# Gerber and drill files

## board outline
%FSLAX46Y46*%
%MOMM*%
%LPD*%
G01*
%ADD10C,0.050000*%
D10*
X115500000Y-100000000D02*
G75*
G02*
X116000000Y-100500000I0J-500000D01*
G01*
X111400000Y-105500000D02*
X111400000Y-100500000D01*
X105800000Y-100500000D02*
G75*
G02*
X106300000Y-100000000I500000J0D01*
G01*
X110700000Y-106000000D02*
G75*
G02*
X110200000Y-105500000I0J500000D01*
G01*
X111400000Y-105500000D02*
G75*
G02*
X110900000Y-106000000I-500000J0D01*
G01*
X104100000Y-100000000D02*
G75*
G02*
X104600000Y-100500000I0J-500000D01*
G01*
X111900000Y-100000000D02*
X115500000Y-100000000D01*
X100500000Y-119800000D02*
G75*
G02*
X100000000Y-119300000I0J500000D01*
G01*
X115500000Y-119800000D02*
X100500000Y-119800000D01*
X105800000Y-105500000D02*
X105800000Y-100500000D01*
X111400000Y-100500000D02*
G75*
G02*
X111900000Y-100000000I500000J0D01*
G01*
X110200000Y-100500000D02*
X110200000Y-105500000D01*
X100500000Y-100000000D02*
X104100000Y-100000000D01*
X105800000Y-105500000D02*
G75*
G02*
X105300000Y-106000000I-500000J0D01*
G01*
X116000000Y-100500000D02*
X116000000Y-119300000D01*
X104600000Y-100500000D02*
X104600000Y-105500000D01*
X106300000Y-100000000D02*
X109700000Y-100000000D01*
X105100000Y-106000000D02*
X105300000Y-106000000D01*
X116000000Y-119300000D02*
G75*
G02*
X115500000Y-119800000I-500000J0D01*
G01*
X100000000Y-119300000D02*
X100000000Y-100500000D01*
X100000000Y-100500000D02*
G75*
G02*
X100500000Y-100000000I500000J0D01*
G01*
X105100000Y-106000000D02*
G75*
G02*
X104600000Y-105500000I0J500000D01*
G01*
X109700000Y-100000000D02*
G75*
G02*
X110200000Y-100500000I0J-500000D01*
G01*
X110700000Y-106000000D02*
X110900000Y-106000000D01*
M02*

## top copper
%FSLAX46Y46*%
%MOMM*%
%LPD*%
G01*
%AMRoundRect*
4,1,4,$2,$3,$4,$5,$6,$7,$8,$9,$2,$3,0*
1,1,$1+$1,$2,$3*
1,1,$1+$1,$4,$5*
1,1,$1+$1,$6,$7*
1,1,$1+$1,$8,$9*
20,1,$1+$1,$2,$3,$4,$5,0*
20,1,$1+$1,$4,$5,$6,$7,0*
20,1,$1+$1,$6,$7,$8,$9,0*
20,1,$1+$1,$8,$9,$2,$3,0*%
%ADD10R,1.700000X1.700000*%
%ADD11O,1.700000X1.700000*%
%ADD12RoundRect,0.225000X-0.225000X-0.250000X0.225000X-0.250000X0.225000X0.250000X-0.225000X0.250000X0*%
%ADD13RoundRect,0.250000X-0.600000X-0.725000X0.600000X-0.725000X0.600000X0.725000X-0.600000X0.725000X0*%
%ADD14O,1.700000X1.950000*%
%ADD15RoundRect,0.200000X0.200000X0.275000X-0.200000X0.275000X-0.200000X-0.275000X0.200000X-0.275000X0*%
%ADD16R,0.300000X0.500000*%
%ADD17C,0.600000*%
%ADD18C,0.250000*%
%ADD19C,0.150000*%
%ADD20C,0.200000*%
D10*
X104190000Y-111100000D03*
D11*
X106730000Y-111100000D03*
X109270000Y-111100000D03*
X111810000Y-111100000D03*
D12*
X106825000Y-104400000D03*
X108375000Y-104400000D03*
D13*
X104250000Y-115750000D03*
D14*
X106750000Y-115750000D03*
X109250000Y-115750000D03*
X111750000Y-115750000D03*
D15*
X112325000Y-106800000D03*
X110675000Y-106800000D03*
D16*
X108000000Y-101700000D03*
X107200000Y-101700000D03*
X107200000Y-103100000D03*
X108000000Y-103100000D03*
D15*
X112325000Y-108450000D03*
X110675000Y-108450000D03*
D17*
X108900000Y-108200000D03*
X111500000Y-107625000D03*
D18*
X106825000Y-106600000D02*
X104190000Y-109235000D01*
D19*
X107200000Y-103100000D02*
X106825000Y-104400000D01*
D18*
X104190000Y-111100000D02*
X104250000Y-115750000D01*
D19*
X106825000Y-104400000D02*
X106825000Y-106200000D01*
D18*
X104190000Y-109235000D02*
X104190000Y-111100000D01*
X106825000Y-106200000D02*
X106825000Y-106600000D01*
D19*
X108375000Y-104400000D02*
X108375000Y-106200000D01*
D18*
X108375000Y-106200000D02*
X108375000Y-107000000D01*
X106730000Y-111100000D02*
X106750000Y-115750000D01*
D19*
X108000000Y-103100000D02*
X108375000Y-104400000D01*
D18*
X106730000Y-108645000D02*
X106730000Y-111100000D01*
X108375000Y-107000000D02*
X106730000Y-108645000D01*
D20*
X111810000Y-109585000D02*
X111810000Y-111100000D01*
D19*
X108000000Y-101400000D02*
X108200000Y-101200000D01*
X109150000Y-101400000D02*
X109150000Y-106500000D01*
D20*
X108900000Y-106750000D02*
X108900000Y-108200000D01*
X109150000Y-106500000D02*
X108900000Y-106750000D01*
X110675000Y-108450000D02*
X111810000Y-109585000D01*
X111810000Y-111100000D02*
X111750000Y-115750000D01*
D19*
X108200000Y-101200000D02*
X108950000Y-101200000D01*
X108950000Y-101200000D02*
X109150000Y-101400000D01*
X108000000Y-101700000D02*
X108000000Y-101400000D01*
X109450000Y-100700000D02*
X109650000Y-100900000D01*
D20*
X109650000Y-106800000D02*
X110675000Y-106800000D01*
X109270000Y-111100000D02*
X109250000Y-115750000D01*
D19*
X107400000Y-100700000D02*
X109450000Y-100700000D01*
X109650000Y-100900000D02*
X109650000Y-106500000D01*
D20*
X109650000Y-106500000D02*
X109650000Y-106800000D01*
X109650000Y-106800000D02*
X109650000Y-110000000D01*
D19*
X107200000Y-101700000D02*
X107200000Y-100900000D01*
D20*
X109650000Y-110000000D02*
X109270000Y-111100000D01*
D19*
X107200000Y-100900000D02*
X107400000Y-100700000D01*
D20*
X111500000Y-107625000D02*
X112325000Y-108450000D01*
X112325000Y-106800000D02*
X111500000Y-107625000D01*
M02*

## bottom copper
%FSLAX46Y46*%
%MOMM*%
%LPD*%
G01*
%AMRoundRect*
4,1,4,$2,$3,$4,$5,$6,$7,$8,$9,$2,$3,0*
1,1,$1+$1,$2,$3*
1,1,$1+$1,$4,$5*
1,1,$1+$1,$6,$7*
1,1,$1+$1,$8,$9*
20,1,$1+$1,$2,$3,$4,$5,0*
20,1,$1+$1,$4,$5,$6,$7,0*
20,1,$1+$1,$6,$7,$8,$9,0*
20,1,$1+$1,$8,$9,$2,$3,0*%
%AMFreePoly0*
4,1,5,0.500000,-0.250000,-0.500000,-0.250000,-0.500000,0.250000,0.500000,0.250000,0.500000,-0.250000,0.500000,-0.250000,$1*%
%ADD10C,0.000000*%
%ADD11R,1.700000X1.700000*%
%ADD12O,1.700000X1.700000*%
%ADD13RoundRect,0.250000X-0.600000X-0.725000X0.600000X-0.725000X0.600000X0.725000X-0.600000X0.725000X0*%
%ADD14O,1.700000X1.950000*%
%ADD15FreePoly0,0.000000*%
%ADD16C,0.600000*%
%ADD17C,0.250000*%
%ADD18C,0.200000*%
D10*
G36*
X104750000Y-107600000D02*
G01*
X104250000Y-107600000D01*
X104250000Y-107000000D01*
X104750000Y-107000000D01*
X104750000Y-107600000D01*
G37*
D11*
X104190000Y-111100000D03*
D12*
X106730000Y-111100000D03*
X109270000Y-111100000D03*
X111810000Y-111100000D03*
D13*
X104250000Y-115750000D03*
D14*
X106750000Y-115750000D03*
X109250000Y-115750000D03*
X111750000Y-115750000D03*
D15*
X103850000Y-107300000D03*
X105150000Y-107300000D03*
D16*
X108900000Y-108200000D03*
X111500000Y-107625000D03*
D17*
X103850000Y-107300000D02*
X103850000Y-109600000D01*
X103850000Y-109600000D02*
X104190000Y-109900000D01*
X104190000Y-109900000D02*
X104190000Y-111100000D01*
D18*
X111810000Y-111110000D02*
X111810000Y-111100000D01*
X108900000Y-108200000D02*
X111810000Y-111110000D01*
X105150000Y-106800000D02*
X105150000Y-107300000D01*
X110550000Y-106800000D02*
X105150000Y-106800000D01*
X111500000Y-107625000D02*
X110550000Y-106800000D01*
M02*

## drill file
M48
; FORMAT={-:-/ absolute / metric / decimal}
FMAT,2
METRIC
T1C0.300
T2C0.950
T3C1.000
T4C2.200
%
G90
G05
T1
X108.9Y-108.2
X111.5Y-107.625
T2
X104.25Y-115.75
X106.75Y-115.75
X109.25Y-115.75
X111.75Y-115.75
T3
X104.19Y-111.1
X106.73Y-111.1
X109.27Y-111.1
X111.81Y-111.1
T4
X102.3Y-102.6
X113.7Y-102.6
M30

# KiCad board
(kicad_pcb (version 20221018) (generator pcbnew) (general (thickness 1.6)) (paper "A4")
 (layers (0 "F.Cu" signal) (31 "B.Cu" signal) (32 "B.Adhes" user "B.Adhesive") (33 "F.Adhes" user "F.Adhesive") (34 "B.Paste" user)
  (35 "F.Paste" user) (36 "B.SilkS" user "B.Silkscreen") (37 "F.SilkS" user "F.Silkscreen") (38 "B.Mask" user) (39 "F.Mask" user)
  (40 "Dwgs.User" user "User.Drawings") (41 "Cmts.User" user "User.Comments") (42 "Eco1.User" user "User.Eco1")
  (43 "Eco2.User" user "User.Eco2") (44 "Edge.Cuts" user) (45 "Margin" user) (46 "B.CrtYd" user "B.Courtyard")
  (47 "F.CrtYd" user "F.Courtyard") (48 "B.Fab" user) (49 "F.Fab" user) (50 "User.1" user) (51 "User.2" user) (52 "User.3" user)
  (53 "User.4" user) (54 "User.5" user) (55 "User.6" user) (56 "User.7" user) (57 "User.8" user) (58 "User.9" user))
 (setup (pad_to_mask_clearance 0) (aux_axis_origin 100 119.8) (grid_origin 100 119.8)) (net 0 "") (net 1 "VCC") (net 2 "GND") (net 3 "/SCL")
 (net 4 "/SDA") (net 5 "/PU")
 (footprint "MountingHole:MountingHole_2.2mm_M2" (layer "F.Cu") (at 113.7 102.6)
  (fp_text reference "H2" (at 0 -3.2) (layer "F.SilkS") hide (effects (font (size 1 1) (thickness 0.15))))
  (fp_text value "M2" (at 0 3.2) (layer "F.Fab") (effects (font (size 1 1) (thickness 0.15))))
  (pad "" np_thru_hole circle (at 0 0) (size 2.2 2.2) (drill 2.2) (layers "*.Cu" "*.Mask")))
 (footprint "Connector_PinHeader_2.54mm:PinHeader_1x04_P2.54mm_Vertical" (layer "F.Cu") (at 104.19 111.1 90)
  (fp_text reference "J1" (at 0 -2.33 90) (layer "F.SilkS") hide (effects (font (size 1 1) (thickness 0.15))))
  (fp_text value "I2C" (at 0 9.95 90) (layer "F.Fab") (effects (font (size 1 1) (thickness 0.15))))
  (pad "1" thru_hole rect (at 0 0 90) (size 1.7 1.7) (drill 1) (layers "*.Cu" "*.Mask") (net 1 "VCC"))
  (pad "2" thru_hole oval (at 0 2.54 90) (size 1.7 1.7) (drill 1) (layers "*.Cu" "*.Mask") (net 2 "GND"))
  (pad "3" thru_hole oval (at 0 5.08 90) (size 1.7 1.7) (drill 1) (layers "*.Cu" "*.Mask") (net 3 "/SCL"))
  (pad "4" thru_hole oval (at 0 7.62 90) (size 1.7 1.7) (drill 1) (layers "*.Cu" "*.Mask") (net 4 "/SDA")))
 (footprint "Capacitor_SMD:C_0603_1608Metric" (layer "F.Cu") (at 107.6 104.4)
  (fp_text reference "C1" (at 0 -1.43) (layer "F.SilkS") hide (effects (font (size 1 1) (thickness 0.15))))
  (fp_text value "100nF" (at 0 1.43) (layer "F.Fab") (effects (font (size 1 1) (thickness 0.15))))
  (pad "1" smd roundrect (at -0.775 0) (size 0.9 0.95) (layers "F.Cu" "F.Paste" "F.Mask") (roundrect_rratio 0.25) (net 1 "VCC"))
  (pad "2" smd roundrect (at 0.775 0) (size 0.9 0.95) (layers "F.Cu" "F.Paste" "F.Mask") (roundrect_rratio 0.25) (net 2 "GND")))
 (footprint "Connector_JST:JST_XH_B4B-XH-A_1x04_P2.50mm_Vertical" (layer "F.Cu") (at 104.25 115.75)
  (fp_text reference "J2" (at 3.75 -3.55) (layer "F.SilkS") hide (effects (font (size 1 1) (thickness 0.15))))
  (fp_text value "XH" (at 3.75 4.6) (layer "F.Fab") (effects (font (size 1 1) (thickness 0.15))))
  (pad "1" thru_hole roundrect (at 0 0) (size 1.7 1.95) (drill 0.95) (layers "*.Cu" "*.Mask") (roundrect_rratio 0.147059) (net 1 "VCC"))
  (pad "2" thru_hole oval (at 2.5 0) (size 1.7 1.95) (drill 0.95) (layers "*.Cu" "*.Mask") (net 2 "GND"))
  (pad "3" thru_hole oval (at 5 0) (size 1.7 1.95) (drill 0.95) (layers "*.Cu" "*.Mask") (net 3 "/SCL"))
  (pad "4" thru_hole oval (at 7.5 0) (size 1.7 1.95) (drill 0.95) (layers "*.Cu" "*.Mask") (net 4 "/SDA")))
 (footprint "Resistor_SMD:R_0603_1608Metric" (layer "F.Cu") (at 111.5 106.8 180)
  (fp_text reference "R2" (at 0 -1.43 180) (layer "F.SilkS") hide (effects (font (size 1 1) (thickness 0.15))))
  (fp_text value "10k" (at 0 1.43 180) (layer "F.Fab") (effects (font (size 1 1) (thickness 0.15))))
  (pad "1" smd roundrect (at -0.825 0 180) (size 0.8 0.95) (layers "F.Cu" "F.Paste" "F.Mask") (roundrect_rratio 0.25) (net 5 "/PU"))
  (pad "2" smd roundrect (at 0.825 0 180) (size 0.8 0.95) (layers "F.Cu" "F.Paste" "F.Mask") (roundrect_rratio 0.25) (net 3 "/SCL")))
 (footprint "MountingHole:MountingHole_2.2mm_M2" (layer "F.Cu") (at 102.3 102.6)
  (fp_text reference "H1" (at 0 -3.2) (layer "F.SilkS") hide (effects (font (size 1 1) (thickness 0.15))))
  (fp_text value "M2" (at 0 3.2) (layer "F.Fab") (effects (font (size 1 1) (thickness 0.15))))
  (pad "" np_thru_hole circle (at 0 0) (size 2.2 2.2) (drill 2.2) (layers "*.Cu" "*.Mask")))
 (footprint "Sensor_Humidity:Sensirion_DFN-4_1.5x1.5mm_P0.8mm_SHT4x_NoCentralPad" (layer "F.Cu") (at 107.6 102.4 -90)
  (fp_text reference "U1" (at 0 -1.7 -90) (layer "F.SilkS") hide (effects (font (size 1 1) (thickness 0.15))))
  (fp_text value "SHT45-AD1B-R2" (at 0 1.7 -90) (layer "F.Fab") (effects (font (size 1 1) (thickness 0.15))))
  (pad "1" smd rect (at -0.7 -0.4 270) (size 0.5 0.3) (layers "F.Cu" "F.Paste" "F.Mask") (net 4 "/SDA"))
  (pad "2" smd rect (at -0.7 0.4 270) (size 0.5 0.3) (layers "F.Cu" "F.Paste" "F.Mask") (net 3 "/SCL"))
  (pad "3" smd rect (at 0.7 0.4 270) (size 0.5 0.3) (layers "F.Cu" "F.Paste" "F.Mask") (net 1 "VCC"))
  (pad "4" smd rect (at 0.7 -0.4 270) (size 0.5 0.3) (layers "F.Cu" "F.Paste" "F.Mask") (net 2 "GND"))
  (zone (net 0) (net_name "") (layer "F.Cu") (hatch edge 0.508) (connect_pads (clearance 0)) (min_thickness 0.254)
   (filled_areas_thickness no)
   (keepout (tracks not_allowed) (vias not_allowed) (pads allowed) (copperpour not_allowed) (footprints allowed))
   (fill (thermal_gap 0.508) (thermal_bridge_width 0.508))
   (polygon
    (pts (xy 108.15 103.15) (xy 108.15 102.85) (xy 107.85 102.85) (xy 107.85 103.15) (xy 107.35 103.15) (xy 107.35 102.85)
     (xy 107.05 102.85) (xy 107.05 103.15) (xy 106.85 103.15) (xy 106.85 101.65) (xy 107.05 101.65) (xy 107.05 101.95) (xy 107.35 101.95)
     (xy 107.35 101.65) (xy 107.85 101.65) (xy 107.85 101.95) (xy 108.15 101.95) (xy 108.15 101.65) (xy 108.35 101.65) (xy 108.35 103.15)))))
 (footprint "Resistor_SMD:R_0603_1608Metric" (layer "F.Cu") (at 111.5 108.45 180)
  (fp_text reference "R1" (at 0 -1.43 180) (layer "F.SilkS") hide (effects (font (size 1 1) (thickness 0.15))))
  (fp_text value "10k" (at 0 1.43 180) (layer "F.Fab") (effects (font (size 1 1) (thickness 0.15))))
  (pad "1" smd roundrect (at -0.825 0 180) (size 0.8 0.95) (layers "F.Cu" "F.Paste" "F.Mask") (roundrect_rratio 0.25) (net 5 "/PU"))
  (pad "2" smd roundrect (at 0.825 0 180) (size 0.8 0.95) (layers "F.Cu" "F.Paste" "F.Mask") (roundrect_rratio 0.25) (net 4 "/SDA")))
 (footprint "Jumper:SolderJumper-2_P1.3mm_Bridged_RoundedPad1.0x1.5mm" (layer "B.Cu") (at 104.5 107.3) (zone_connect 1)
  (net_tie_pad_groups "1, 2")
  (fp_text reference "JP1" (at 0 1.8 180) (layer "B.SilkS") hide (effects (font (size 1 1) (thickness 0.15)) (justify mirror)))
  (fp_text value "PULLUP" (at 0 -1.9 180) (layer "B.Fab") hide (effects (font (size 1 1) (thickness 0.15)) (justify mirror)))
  (fp_poly (pts (xy 0.25 0.3) (xy -0.25 0.3) (xy -0.25 -0.3) (xy 0.25 -0.3)) (stroke (width 0) (type solid)) (fill solid) (layer "B.Cu"))
  (pad "1" smd custom (at -0.65 0) (size 1 0.5) (layers "B.Cu" "B.Mask") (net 1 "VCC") (zone_connect 2) (thermal_bridge_angle 45)
   (options (clearance outline) (anchor rect)) (primitives))
  (pad "2" smd custom (at 0.65 0) (size 1 0.5) (layers "B.Cu" "B.Mask") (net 5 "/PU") (zone_connect 2) (thermal_bridge_angle 45)
   (options (clearance outline) (anchor rect)) (primitives)))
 (gr_arc (start 115.5 100) (mid 115.853553 100.146446) (end 116 100.5) (stroke (width 0.05) (type default)) (layer "Edge.Cuts"))
 (gr_line (start 111.4 105.5) (end 111.4 100.5) (stroke (width 0.05) (type default)) (layer "Edge.Cuts"))
 (gr_arc (start 105.8 100.5) (mid 105.946446 100.146446) (end 106.3 100) (stroke (width 0.05) (type default)) (layer "Edge.Cuts"))
 (gr_arc (start 110.7 106) (mid 110.346447 105.853553) (end 110.2 105.5) (stroke (width 0.05) (type default)) (layer "Edge.Cuts"))
 (gr_arc (start 111.4 105.5) (mid 111.253553 105.853553) (end 110.9 106) (stroke (width 0.05) (type default)) (layer "Edge.Cuts"))
 (gr_arc (start 104.1 100) (mid 104.453553 100.146446) (end 104.6 100.5) (stroke (width 0.05) (type default)) (layer "Edge.Cuts"))
 (gr_line (start 111.9 100) (end 115.5 100) (stroke (width 0.05) (type default)) (layer "Edge.Cuts"))
 (gr_arc (start 100.5 119.8) (mid 100.146446 119.653553) (end 100 119.3) (stroke (width 0.05) (type default)) (layer "Edge.Cuts"))
 (gr_line (start 115.5 119.8) (end 100.5 119.8) (stroke (width 0.05) (type default)) (layer "Edge.Cuts"))
 (gr_line (start 105.8 105.5) (end 105.8 100.5) (stroke (width 0.05) (type default)) (layer "Edge.Cuts"))
 (gr_arc (start 111.4 100.5) (mid 111.546446 100.146446) (end 111.9 100) (stroke (width 0.05) (type default)) (layer "Edge.Cuts"))
 (gr_line (start 110.2 100.5) (end 110.2 105.5) (stroke (width 0.05) (type default)) (layer "Edge.Cuts"))
 (gr_line (start 100.5 100) (end 104.1 100) (stroke (width 0.05) (type default)) (layer "Edge.Cuts"))
 (gr_arc (start 105.8 105.5) (mid 105.653553 105.853553) (end 105.3 106) (stroke (width 0.05) (type default)) (layer "Edge.Cuts"))
 (gr_line (start 116 100.5) (end 116 119.3) (stroke (width 0.05) (type default)) (layer "Edge.Cuts"))
 (gr_line (start 104.6 100.5) (end 104.6 105.5) (stroke (width 0.05) (type default)) (layer "Edge.Cuts"))
 (gr_line (start 106.3 100) (end 109.7 100) (stroke (width 0.05) (type default)) (layer "Edge.Cuts"))
 (gr_line (start 105.1 106) (end 105.3 106) (stroke (width 0.05) (type default)) (layer "Edge.Cuts"))
 (gr_arc (start 116 119.3) (mid 115.853553 119.653553) (end 115.5 119.8) (stroke (width 0.05) (type default)) (layer "Edge.Cuts"))
 (gr_line (start 100 119.3) (end 100 100.5) (stroke (width 0.05) (type default)) (layer "Edge.Cuts"))
 (gr_arc (start 100 100.5) (mid 100.146446 100.146446) (end 100.5 100) (stroke (width 0.05) (type default)) (layer "Edge.Cuts"))
 (gr_arc (start 105.1 106) (mid 104.746447 105.853553) (end 104.6 105.5) (stroke (width 0.05) (type default)) (layer "Edge.Cuts"))
 (gr_arc (start 109.7 100) (mid 110.053553 100.146446) (end 110.2 100.5) (stroke (width 0.05) (type default)) (layer "Edge.Cuts"))
 (gr_line (start 110.7 106) (end 110.9 106) (stroke (width 0.05) (type default)) (layer "Edge.Cuts"))
 (segment (start 106.825 106.6) (end 104.19 109.235) (width 0.25) (layer "F.Cu") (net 1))
 (segment (start 107.2 103.1) (end 106.825 104.4) (width 0.15) (layer "F.Cu") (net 1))
 (segment (start 104.19 111.1) (end 104.25 115.75) (width 0.25) (layer "F.Cu") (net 1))
 (segment (start 106.825 104.4) (end 106.825 106.2) (width 0.15) (layer "F.Cu") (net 1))
 (segment (start 104.19 109.235) (end 104.19 111.1) (width 0.25) (layer "F.Cu") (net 1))
 (segment (start 106.825 106.2) (end 106.825 106.6) (width 0.25) (layer "F.Cu") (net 1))
 (segment (start 103.85 107.3) (end 103.85 109.6) (width 0.25) (layer "B.Cu") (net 1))
 (segment (start 103.85 109.6) (end 104.19 109.9) (width 0.25) (layer "B.Cu") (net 1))
 (segment (start 104.19 109.9) (end 104.19 111.1) (width 0.25) (layer "B.Cu") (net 1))
 (segment (start 108.375 104.4) (end 108.375 106.2) (width 0.15) (layer "F.Cu") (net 2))
 (segment (start 108.375 106.2) (end 108.375 107) (width 0.25) (layer "F.Cu") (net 2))
 (segment (start 106.73 111.1) (end 106.75 115.75) (width 0.25) (layer "F.Cu") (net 2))
 (segment (start 108 103.1) (end 108.375 104.4) (width 0.15) (layer "F.Cu") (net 2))
 (segment (start 106.73 108.645) (end 106.73 111.1) (width 0.25) (layer "F.Cu") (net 2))
 (segment (start 108.375 107) (end 106.73 108.645) (width 0.25) (layer "F.Cu") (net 2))
 (segment (start 111.81 109.585) (end 111.81 111.1) (width 0.2) (layer "F.Cu") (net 4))
 (segment (start 108 101.4) (end 108.2 101.2) (width 0.15) (layer "F.Cu") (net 4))
 (segment (start 109.15 101.4) (end 109.15 106.5) (width 0.15) (layer "F.Cu") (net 4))
 (segment (start 108.9 106.75) (end 108.9 108.2) (width 0.2) (layer "F.Cu") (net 4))
 (segment (start 109.15 106.5) (end 108.9 106.75) (width 0.2) (layer "F.Cu") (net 4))
 (segment (start 110.675 108.45) (end 111.81 109.585) (width 0.2) (layer "F.Cu") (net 4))
 (segment (start 111.81 111.1) (end 111.75 115.75) (width 0.2) (layer "F.Cu") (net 4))
 (segment (start 108.2 101.2) (end 108.95 101.2) (width 0.15) (layer "F.Cu") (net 4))
 (segment (start 108.95 101.2) (end 109.15 101.4) (width 0.15) (layer "F.Cu") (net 4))
 (segment (start 108 101.7) (end 108 101.4) (width 0.15) (layer "F.Cu") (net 4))
 (via (at 108.9 108.2) (size 0.6) (drill 0.3) (layers "F.Cu" "B.Cu") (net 4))
 (segment (start 111.81 111.11) (end 111.81 111.1) (width 0.2) (layer "B.Cu") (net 4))
 (segment (start 108.9 108.2) (end 111.81 111.11) (width 0.2) (layer "B.Cu") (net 4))
 (segment (start 109.45 100.7) (end 109.65 100.9) (width 0.15) (layer "F.Cu") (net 3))
 (segment (start 109.65 106.8) (end 110.675 106.8) (width 0.2) (layer "F.Cu") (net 3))
 (segment (start 109.27 111.1) (end 109.25 115.75) (width 0.2) (layer "F.Cu") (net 3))
 (segment (start 107.4 100.7) (end 109.45 100.7) (width 0.15) (layer "F.Cu") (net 3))
 (segment (start 109.65 100.9) (end 109.65 106.5) (width 0.15) (layer "F.Cu") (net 3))
 (segment (start 109.65 106.5) (end 109.65 106.8) (width 0.2) (layer "F.Cu") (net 3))
 (segment (start 109.65 106.8) (end 109.65 110) (width 0.2) (layer "F.Cu") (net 3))
 (segment (start 107.2 101.7) (end 107.2 100.9) (width 0.15) (layer "F.Cu") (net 3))
 (segment (start 109.65 110) (end 109.27 111.1) (width 0.2) (layer "F.Cu") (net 3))
 (segment (start 107.2 100.9) (end 107.4 100.7) (width 0.15) (layer "F.Cu") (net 3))
 (segment (start 111.5 107.625) (end 112.325 108.45) (width 0.2) (layer "F.Cu") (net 5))
 (segment (start 112.325 106.8) (end 111.5 107.625) (width 0.2) (layer "F.Cu") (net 5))
 (via (at 111.5 107.625) (size 0.6) (drill 0.3) (layers "F.Cu" "B.Cu") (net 5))
 (segment (start 105.15 106.8) (end 105.15 107.3) (width 0.2) (layer "B.Cu") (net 5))
 (segment (start 110.55 106.8) (end 105.15 106.8) (width 0.2) (layer "B.Cu") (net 5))
 (segment (start 111.5 107.625) (end 110.55 106.8) (width 0.2) (layer "B.Cu") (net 5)))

